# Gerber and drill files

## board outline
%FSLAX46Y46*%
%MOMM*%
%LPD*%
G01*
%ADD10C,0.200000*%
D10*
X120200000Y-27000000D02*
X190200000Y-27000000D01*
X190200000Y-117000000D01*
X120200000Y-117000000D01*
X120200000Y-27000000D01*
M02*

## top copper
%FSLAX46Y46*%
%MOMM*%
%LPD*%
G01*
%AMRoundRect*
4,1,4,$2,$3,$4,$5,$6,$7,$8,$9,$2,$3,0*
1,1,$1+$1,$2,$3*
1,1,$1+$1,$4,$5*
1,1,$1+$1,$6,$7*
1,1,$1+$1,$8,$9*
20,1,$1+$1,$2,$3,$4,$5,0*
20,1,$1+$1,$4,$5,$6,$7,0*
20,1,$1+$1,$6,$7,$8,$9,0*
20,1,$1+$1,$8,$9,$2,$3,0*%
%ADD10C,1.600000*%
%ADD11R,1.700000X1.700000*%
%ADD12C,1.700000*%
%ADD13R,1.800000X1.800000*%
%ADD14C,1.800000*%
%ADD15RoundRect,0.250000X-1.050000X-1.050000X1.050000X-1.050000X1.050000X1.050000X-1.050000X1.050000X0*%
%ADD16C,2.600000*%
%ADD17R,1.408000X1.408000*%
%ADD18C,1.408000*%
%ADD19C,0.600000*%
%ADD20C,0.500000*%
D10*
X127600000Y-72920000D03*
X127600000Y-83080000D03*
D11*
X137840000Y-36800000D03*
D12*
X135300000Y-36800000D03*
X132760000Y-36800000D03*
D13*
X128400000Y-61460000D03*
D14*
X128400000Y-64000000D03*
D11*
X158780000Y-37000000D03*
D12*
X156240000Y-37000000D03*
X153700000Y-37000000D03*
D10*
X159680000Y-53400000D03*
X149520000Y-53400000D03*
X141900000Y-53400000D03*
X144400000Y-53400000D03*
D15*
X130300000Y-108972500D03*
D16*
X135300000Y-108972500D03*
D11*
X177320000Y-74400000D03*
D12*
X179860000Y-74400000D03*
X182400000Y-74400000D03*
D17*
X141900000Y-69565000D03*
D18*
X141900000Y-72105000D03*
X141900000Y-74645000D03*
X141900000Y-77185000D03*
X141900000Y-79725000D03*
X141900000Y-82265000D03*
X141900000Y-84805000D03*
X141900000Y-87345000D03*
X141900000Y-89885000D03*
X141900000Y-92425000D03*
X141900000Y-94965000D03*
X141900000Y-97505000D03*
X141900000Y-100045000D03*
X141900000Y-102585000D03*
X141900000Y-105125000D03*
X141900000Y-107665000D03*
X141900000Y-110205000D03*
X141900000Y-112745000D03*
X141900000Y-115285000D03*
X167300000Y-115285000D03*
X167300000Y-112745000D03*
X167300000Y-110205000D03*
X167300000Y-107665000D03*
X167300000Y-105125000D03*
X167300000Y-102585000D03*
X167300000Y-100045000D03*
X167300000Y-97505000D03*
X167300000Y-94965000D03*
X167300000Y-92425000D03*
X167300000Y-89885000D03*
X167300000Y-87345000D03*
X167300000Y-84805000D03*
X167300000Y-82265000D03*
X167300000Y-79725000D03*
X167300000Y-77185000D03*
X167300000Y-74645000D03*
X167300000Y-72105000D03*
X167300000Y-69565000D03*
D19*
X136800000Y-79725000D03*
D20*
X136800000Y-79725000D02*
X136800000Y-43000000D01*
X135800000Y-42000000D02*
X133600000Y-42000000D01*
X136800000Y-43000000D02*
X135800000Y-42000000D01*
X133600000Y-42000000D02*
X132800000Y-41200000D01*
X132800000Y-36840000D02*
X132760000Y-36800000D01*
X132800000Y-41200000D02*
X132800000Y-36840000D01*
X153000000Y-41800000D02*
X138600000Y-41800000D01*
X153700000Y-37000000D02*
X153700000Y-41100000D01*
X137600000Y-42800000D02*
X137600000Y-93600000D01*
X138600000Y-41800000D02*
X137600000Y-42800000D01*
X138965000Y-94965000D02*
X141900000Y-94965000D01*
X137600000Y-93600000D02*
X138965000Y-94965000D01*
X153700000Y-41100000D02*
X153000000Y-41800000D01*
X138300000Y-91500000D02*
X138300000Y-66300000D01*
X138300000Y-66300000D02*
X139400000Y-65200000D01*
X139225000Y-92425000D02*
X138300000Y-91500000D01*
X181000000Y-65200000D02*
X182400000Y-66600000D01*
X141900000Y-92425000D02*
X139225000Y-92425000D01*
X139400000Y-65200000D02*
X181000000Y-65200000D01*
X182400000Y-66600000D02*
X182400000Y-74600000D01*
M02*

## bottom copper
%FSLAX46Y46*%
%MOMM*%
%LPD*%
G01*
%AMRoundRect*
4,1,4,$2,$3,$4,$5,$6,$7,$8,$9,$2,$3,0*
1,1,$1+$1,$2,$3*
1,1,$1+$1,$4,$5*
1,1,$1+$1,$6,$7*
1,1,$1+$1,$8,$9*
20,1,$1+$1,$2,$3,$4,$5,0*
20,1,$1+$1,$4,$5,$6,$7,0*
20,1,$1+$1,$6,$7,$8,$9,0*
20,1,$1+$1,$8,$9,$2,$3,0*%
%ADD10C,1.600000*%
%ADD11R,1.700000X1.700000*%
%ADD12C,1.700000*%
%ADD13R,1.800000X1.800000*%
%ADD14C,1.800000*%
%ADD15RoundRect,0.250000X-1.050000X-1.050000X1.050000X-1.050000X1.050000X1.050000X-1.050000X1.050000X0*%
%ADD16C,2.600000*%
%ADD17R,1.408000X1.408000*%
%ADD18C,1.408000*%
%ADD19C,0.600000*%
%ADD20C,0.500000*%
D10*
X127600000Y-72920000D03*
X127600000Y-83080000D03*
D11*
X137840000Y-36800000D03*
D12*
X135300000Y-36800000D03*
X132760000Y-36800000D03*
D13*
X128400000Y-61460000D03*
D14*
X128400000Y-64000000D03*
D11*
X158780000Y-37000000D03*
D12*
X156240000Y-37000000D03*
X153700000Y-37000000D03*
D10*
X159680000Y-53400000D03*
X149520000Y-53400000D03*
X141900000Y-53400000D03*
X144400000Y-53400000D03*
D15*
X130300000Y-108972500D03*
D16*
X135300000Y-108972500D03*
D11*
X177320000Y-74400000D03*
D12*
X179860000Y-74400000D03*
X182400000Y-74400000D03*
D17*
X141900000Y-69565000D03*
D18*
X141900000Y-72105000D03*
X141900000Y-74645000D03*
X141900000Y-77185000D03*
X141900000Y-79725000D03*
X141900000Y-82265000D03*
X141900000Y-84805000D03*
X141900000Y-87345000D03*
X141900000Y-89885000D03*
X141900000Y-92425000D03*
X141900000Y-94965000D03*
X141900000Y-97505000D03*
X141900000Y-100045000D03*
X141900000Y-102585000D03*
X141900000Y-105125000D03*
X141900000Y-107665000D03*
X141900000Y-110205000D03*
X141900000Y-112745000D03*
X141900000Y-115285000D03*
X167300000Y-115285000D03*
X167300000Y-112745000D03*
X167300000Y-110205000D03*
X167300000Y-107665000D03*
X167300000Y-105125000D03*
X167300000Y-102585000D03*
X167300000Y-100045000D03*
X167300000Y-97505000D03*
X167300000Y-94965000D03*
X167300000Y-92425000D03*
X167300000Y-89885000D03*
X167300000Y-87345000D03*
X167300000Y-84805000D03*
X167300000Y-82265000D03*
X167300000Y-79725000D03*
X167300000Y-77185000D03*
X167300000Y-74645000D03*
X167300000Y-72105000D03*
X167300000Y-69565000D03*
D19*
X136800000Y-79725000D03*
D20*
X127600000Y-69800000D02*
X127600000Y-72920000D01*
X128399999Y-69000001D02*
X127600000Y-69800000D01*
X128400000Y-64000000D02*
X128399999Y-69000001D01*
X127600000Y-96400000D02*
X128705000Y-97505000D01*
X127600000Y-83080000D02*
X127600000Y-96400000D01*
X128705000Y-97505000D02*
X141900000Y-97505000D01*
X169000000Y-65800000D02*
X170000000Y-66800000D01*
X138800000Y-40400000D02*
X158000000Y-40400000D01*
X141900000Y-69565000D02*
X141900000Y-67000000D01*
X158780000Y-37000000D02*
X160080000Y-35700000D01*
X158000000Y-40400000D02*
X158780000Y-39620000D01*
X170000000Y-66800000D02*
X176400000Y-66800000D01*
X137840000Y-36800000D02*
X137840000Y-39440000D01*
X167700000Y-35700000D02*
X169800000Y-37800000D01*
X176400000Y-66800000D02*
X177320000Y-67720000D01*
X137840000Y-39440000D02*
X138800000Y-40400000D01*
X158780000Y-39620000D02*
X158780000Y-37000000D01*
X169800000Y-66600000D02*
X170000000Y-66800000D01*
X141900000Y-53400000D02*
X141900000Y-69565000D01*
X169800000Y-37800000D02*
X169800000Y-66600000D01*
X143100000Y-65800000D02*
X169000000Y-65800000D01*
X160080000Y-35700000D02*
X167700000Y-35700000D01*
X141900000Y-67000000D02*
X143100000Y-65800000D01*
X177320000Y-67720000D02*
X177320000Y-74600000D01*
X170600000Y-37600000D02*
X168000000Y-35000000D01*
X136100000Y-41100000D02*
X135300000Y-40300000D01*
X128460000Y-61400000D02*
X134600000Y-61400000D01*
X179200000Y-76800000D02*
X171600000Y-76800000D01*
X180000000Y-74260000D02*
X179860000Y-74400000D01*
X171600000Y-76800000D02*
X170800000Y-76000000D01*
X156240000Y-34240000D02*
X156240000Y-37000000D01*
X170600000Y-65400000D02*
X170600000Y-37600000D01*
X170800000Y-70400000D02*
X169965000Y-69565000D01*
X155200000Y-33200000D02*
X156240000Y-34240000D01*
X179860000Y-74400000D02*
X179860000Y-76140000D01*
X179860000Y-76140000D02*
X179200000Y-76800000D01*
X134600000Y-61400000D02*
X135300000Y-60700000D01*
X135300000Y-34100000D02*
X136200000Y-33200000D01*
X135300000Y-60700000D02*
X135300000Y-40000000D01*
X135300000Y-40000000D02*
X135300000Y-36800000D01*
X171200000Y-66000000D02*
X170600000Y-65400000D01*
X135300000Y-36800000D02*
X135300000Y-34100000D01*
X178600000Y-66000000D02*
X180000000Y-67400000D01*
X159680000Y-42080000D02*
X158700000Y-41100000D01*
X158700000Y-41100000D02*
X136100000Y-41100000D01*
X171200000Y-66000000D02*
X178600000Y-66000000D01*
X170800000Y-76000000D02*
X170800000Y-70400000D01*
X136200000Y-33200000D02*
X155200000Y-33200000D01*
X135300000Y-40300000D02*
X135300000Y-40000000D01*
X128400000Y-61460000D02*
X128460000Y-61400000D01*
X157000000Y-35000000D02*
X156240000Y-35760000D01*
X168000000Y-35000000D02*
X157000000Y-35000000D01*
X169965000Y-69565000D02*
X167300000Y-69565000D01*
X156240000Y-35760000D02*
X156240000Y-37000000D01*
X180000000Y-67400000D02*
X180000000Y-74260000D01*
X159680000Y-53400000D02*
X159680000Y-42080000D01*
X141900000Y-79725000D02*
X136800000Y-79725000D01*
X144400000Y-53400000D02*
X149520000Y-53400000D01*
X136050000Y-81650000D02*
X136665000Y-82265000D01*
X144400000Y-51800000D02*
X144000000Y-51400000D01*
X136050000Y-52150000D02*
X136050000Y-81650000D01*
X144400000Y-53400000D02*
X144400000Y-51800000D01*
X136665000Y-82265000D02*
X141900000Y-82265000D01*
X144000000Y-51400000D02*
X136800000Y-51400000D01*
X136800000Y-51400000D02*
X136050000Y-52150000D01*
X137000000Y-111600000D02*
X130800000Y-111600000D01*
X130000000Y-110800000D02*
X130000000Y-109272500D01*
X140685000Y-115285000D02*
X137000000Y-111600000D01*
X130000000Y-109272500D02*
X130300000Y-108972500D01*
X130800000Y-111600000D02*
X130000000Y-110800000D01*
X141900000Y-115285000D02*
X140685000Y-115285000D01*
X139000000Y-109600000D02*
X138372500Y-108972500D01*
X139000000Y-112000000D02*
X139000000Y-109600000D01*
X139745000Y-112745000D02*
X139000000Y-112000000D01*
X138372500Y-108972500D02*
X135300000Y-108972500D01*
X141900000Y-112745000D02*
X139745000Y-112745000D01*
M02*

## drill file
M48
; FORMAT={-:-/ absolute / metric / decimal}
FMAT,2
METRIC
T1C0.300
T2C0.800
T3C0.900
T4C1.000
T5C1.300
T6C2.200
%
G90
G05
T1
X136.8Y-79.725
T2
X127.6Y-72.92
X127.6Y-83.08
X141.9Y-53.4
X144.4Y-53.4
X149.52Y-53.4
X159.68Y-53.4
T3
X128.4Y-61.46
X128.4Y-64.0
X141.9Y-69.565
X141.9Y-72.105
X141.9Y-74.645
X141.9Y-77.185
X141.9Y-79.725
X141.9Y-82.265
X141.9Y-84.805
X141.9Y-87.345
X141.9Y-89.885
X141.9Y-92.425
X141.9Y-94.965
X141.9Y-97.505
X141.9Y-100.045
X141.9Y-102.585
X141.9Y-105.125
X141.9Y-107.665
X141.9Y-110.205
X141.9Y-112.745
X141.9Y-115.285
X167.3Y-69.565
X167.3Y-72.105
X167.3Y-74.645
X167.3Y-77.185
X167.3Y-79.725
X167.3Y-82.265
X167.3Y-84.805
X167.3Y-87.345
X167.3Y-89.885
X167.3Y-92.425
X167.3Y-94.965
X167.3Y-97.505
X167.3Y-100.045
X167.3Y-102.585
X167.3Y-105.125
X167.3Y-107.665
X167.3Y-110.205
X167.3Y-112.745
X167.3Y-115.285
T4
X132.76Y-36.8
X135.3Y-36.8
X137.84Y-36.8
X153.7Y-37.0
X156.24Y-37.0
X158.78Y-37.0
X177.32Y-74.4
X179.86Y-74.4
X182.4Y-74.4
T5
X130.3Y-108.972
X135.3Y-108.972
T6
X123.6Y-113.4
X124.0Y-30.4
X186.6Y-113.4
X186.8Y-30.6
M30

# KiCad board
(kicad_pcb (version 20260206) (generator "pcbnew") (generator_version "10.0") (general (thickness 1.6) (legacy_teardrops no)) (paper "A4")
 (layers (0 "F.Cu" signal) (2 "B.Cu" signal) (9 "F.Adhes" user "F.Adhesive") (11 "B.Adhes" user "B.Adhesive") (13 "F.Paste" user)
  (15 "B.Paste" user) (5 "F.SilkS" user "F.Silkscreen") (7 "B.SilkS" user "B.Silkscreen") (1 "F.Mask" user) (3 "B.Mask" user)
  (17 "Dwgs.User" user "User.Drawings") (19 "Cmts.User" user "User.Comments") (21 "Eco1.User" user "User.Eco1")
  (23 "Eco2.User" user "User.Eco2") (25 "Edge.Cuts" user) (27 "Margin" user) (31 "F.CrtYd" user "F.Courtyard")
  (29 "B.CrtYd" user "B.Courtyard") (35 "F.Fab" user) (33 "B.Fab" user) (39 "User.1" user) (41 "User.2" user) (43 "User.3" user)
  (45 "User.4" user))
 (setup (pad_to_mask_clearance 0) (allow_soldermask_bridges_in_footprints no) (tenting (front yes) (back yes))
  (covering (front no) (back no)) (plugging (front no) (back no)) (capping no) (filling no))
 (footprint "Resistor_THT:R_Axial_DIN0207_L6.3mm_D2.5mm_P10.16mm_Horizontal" (layer "F.Cu") (at 127.6 72.92 -90)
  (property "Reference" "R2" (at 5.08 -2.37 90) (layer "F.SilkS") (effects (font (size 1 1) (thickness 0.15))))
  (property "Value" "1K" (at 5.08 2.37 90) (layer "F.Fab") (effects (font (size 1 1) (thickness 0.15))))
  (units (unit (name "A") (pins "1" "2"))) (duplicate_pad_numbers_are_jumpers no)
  (pad "1" thru_hole circle (at 0 0 270) (size 1.6 1.6) (drill 0.8) (layers "*.Cu" "*.Mask") (remove_unused_layers no) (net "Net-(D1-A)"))
  (pad "2" thru_hole circle (at 10.16 0 270) (size 1.6 1.6) (drill 0.8) (layers "*.Cu" "*.Mask") (remove_unused_layers no)
   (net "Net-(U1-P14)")))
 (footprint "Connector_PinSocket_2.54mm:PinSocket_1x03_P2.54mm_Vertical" (layer "F.Cu") (at 137.84 36.8 -90)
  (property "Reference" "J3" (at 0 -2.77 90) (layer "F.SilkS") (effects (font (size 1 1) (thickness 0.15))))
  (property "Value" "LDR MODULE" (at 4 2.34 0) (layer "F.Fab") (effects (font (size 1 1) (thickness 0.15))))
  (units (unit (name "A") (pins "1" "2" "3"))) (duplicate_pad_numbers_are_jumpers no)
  (pad "1" thru_hole rect (at 0 0 270) (size 1.7 1.7) (drill 1) (layers "*.Cu" "*.Mask") (remove_unused_layers no) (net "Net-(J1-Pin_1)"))
  (pad "2" thru_hole circle (at 0 2.54 270) (size 1.7 1.7) (drill 1) (layers "*.Cu" "*.Mask") (remove_unused_layers no) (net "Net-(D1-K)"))
  (pad "3" thru_hole circle (at 0 5.08 270) (size 1.7 1.7) (drill 1) (layers "*.Cu" "*.Mask") (remove_unused_layers no) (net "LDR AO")))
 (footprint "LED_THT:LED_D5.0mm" (layer "F.Cu") (at 128.4 61.46 -90)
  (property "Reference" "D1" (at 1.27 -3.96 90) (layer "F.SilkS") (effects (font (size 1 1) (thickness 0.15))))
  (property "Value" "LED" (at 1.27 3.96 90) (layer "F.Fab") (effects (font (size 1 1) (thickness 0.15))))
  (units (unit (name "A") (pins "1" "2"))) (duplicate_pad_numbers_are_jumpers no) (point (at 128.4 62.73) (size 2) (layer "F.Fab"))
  (pad "1" thru_hole rect (at 0 0 270) (size 1.8 1.8) (drill 0.9) (layers "*.Cu" "*.Mask") (remove_unused_layers no) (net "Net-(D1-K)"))
  (pad "2" thru_hole circle (at 2.54 0 270) (size 1.8 1.8) (drill 0.9) (layers "*.Cu" "*.Mask") (remove_unused_layers no) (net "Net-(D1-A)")))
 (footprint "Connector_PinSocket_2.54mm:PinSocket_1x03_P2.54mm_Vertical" (layer "F.Cu") (at 158.78 37 -90)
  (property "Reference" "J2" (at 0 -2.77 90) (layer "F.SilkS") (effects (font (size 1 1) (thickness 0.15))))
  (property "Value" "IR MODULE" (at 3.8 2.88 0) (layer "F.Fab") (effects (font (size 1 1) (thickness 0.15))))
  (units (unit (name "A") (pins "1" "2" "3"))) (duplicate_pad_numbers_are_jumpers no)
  (pad "1" thru_hole rect (at 0 0 270) (size 1.7 1.7) (drill 1) (layers "*.Cu" "*.Mask") (remove_unused_layers no) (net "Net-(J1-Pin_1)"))
  (pad "2" thru_hole circle (at 0 2.54 270) (size 1.7 1.7) (drill 1) (layers "*.Cu" "*.Mask") (remove_unused_layers no) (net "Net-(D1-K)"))
  (pad "3" thru_hole circle (at 0 5.08 270) (size 1.7 1.7) (drill 1) (layers "*.Cu" "*.Mask") (remove_unused_layers no) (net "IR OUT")))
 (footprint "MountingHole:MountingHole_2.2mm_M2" (layer "F.Cu") (at 186.6 113.4)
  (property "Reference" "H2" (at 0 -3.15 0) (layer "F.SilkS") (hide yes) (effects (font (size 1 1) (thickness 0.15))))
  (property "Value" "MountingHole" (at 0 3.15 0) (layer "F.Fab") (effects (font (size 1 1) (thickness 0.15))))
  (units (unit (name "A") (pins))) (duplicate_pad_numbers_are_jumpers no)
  (pad "" np_thru_hole circle (at 0 0) (size 2.2 2.2) (drill 2.2) (layers "*.Cu" "*.Mask")))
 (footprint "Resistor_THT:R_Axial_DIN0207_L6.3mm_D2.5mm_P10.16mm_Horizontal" (layer "F.Cu") (at 159.68 53.4 180)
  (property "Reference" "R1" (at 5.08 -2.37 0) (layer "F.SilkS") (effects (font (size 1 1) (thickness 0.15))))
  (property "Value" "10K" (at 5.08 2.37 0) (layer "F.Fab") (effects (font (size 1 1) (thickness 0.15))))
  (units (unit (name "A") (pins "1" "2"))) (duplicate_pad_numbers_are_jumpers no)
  (pad "1" thru_hole circle (at 0 0 180) (size 1.6 1.6) (drill 0.8) (layers "*.Cu" "*.Mask") (remove_unused_layers no) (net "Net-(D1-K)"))
  (pad "2" thru_hole circle (at 10.16 0 180) (size 1.6 1.6) (drill 0.8) (layers "*.Cu" "*.Mask") (remove_unused_layers no) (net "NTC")))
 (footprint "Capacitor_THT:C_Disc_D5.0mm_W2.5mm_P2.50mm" (layer "F.Cu") (at 141.9 53.4)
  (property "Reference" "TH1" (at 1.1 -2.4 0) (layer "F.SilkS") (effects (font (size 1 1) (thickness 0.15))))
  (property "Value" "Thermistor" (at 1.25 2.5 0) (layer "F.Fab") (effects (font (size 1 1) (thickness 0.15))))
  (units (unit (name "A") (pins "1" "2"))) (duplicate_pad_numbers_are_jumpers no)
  (pad "1" thru_hole circle (at 0 0) (size 1.6 1.6) (drill 0.8) (layers "*.Cu" "*.Mask") (remove_unused_layers no) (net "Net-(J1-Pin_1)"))
  (pad "2" thru_hole circle (at 2.5 0) (size 1.6 1.6) (drill 0.8) (layers "*.Cu" "*.Mask") (remove_unused_layers no) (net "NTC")))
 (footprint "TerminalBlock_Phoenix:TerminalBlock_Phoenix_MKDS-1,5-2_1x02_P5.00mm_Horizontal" (layer "F.Cu") (at 130.3 108.9725)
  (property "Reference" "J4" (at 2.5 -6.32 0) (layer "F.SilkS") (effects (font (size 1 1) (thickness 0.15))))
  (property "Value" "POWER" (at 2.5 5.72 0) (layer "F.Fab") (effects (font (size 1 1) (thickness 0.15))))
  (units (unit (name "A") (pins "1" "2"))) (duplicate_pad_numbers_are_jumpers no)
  (pad "1" thru_hole roundrect (at 0 0) (size 2.6 2.6) (drill 1.3) (layers "*.Cu" "*.Mask") (remove_unused_layers no)
   (roundrect_rratio 0.096154) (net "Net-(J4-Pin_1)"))
  (pad "2" thru_hole circle (at 5 0) (size 2.6 2.6) (drill 1.3) (layers "*.Cu" "*.Mask") (remove_unused_layers no) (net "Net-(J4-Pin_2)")))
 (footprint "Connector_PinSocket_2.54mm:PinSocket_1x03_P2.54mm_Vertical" (layer "F.Cu") (at 177.32 74.4 90)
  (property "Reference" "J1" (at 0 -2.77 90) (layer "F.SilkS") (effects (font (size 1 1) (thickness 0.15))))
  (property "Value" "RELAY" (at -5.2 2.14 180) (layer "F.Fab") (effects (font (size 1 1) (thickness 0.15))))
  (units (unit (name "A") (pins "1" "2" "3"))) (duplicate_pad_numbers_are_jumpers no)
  (pad "1" thru_hole rect (at 0 0 90) (size 1.7 1.7) (drill 1) (layers "*.Cu" "*.Mask") (remove_unused_layers no) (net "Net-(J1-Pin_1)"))
  (pad "2" thru_hole circle (at 0 2.54 90) (size 1.7 1.7) (drill 1) (layers "*.Cu" "*.Mask") (remove_unused_layers no) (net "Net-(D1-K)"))
  (pad "3" thru_hole circle (at 0 5.08 90) (size 1.7 1.7) (drill 1) (layers "*.Cu" "*.Mask") (remove_unused_layers no) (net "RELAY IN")))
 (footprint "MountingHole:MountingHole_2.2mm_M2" (layer "F.Cu") (at 186.8 30.6)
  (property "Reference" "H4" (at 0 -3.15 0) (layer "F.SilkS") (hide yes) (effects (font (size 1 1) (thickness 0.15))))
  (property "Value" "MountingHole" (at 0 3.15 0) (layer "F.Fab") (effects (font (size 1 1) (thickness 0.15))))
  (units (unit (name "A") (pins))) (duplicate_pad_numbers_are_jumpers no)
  (pad "" np_thru_hole circle (at 0 0) (size 2.2 2.2) (drill 2.2) (layers "*.Cu" "*.Mask")))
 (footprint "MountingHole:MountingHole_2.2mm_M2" (layer "F.Cu") (at 124 30.4)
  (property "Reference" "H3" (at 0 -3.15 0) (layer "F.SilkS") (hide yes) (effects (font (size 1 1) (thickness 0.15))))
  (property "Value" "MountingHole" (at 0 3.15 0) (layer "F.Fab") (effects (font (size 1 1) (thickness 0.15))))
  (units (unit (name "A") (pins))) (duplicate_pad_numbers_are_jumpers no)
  (pad "" np_thru_hole circle (at 0 0) (size 2.2 2.2) (drill 2.2) (layers "*.Cu" "*.Mask")))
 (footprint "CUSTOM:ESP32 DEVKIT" (layer "F.Cu") (at 154.57 93.21)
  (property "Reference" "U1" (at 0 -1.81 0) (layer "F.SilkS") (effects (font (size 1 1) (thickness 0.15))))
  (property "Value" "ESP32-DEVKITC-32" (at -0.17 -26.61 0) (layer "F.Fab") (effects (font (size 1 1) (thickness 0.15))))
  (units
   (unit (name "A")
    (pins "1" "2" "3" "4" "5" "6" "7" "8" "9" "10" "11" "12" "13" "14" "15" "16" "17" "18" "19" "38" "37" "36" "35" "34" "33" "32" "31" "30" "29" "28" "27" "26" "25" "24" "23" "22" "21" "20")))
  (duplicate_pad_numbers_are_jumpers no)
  (pad "1" thru_hole rect (at -12.67 -23.645) (size 1.408 1.408) (drill 0.9) (layers "*.Cu" "*.Mask") (remove_unused_layers no)
   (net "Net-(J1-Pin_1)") (solder_mask_margin 0.102))
  (pad "2" thru_hole circle (at -12.67 -21.105) (size 1.408 1.408) (drill 0.9) (layers "*.Cu" "*.Mask") (remove_unused_layers no)
   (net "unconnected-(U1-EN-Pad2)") (solder_mask_margin 0.102))
  (pad "3" thru_hole circle (at -12.67 -18.565) (size 1.408 1.408) (drill 0.9) (layers "*.Cu" "*.Mask") (remove_unused_layers no)
   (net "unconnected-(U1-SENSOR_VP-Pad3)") (solder_mask_margin 0.102))
  (pad "4" thru_hole circle (at -12.67 -16.025) (size 1.408 1.408) (drill 0.9) (layers "*.Cu" "*.Mask") (remove_unused_layers no)
   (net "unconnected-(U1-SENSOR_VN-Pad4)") (solder_mask_margin 0.102))
  (pad "5" thru_hole circle (at -12.67 -13.485) (size 1.408 1.408) (drill 0.9) (layers "*.Cu" "*.Mask") (remove_unused_layers no)
   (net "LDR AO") (solder_mask_margin 0.102))
  (pad "6" thru_hole circle (at -12.67 -10.945) (size 1.408 1.408) (drill 0.9) (layers "*.Cu" "*.Mask") (remove_unused_layers no)
   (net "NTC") (solder_mask_margin 0.102))
  (pad "7" thru_hole circle (at -12.67 -8.405) (size 1.408 1.408) (drill 0.9) (layers "*.Cu" "*.Mask") (remove_unused_layers no)
   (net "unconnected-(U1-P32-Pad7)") (solder_mask_margin 0.102))
  (pad "8" thru_hole circle (at -12.67 -5.865) (size 1.408 1.408) (drill 0.9) (layers "*.Cu" "*.Mask") (remove_unused_layers no)
   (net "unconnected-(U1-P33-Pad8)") (solder_mask_margin 0.102))
  (pad "9" thru_hole circle (at -12.67 -3.325) (size 1.408 1.408) (drill 0.9) (layers "*.Cu" "*.Mask") (remove_unused_layers no)
   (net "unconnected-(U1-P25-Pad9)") (solder_mask_margin 0.102))
  (pad "10" thru_hole circle (at -12.67 -0.785) (size 1.408 1.408) (drill 0.9) (layers "*.Cu" "*.Mask") (remove_unused_layers no)
   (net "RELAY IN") (solder_mask_margin 0.102))
  (pad "11" thru_hole circle (at -12.67 1.755) (size 1.408 1.408) (drill 0.9) (layers "*.Cu" "*.Mask") (remove_unused_layers no)
   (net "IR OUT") (solder_mask_margin 0.102))
  (pad "12" thru_hole circle (at -12.67 4.295) (size 1.408 1.408) (drill 0.9) (layers "*.Cu" "*.Mask") (remove_unused_layers no)
   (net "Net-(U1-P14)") (solder_mask_margin 0.102))
  (pad "13" thru_hole circle (at -12.67 6.835) (size 1.408 1.408) (drill 0.9) (layers "*.Cu" "*.Mask") (remove_unused_layers no)
   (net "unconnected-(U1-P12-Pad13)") (solder_mask_margin 0.102))
  (pad "14" thru_hole circle (at -12.67 9.375) (size 1.408 1.408) (drill 0.9) (layers "*.Cu" "*.Mask") (remove_unused_layers no)
   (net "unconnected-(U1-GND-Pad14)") (solder_mask_margin 0.102))
  (pad "15" thru_hole circle (at -12.67 11.915) (size 1.408 1.408) (drill 0.9) (layers "*.Cu" "*.Mask") (remove_unused_layers no)
   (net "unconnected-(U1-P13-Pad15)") (solder_mask_margin 0.102))
  (pad "16" thru_hole circle (at -12.67 14.455) (size 1.408 1.408) (drill 0.9) (layers "*.Cu" "*.Mask") (remove_unused_layers no)
   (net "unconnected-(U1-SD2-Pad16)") (solder_mask_margin 0.102))
  (pad "17" thru_hole circle (at -12.67 16.995) (size 1.408 1.408) (drill 0.9) (layers "*.Cu" "*.Mask") (remove_unused_layers no)
   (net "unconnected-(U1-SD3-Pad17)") (solder_mask_margin 0.102))
  (pad "18" thru_hole circle (at -12.67 19.535) (size 1.408 1.408) (drill 0.9) (layers "*.Cu" "*.Mask") (remove_unused_layers no)
   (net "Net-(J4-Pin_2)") (solder_mask_margin 0.102))
  (pad "19" thru_hole circle (at -12.67 22.075) (size 1.408 1.408) (drill 0.9) (layers "*.Cu" "*.Mask") (remove_unused_layers no)
   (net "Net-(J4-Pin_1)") (solder_mask_margin 0.102))
  (pad "20" thru_hole circle (at 12.73 22.075) (size 1.408 1.408) (drill 0.9) (layers "*.Cu" "*.Mask") (remove_unused_layers no)
   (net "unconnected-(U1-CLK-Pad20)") (solder_mask_margin 0.102))
  (pad "21" thru_hole circle (at 12.73 19.535) (size 1.408 1.408) (drill 0.9) (layers "*.Cu" "*.Mask") (remove_unused_layers no)
   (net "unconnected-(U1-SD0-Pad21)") (solder_mask_margin 0.102))
  (pad "22" thru_hole circle (at 12.73 16.995) (size 1.408 1.408) (drill 0.9) (layers "*.Cu" "*.Mask") (remove_unused_layers no)
   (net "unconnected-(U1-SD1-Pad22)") (solder_mask_margin 0.102))
  (pad "23" thru_hole circle (at 12.73 14.455) (size 1.408 1.408) (drill 0.9) (layers "*.Cu" "*.Mask") (remove_unused_layers no)
   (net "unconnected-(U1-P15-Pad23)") (solder_mask_margin 0.102))
  (pad "24" thru_hole circle (at 12.73 11.915) (size 1.408 1.408) (drill 0.9) (layers "*.Cu" "*.Mask") (remove_unused_layers no)
   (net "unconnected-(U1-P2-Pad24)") (solder_mask_margin 0.102))
  (pad "25" thru_hole circle (at 12.73 9.375) (size 1.408 1.408) (drill 0.9) (layers "*.Cu" "*.Mask") (remove_unused_layers no)
   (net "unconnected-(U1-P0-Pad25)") (solder_mask_margin 0.102))
  (pad "26" thru_hole circle (at 12.73 6.835) (size 1.408 1.408) (drill 0.9) (layers "*.Cu" "*.Mask") (remove_unused_layers no)
   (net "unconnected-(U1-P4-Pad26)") (solder_mask_margin 0.102))
  (pad "27" thru_hole circle (at 12.73 4.295) (size 1.408 1.408) (drill 0.9) (layers "*.Cu" "*.Mask") (remove_unused_layers no)
   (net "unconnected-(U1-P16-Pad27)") (solder_mask_margin 0.102))
  (pad "28" thru_hole circle (at 12.73 1.755) (size 1.408 1.408) (drill 0.9) (layers "*.Cu" "*.Mask") (remove_unused_layers no)
   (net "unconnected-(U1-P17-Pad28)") (solder_mask_margin 0.102))
  (pad "29" thru_hole circle (at 12.73 -0.785) (size 1.408 1.408) (drill 0.9) (layers "*.Cu" "*.Mask") (remove_unused_layers no)
   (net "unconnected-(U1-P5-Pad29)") (solder_mask_margin 0.102))
  (pad "30" thru_hole circle (at 12.73 -3.325) (size 1.408 1.408) (drill 0.9) (layers "*.Cu" "*.Mask") (remove_unused_layers no)
   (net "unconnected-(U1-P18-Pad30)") (solder_mask_margin 0.102))
  (pad "31" thru_hole circle (at 12.73 -5.865) (size 1.408 1.408) (drill 0.9) (layers "*.Cu" "*.Mask") (remove_unused_layers no)
   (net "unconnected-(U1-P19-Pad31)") (solder_mask_margin 0.102))
  (pad "32" thru_hole circle (at 12.73 -8.405) (size 1.408 1.408) (drill 0.9) (layers "*.Cu" "*.Mask") (remove_unused_layers no)
   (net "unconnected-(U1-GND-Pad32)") (solder_mask_margin 0.102))
  (pad "33" thru_hole circle (at 12.73 -10.945) (size 1.408 1.408) (drill 0.9) (layers "*.Cu" "*.Mask") (remove_unused_layers no)
   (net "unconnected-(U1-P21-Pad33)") (solder_mask_margin 0.102))
  (pad "34" thru_hole circle (at 12.73 -13.485) (size 1.408 1.408) (drill 0.9) (layers "*.Cu" "*.Mask") (remove_unused_layers no)
   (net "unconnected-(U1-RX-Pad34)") (solder_mask_margin 0.102))
  (pad "35" thru_hole circle (at 12.73 -16.025) (size 1.408 1.408) (drill 0.9) (layers "*.Cu" "*.Mask") (remove_unused_layers no)
   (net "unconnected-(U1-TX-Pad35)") (solder_mask_margin 0.102))
  (pad "36" thru_hole circle (at 12.73 -18.565) (size 1.408 1.408) (drill 0.9) (layers "*.Cu" "*.Mask") (remove_unused_layers no)
   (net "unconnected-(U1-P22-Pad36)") (solder_mask_margin 0.102))
  (pad "37" thru_hole circle (at 12.73 -21.105) (size 1.408 1.408) (drill 0.9) (layers "*.Cu" "*.Mask") (remove_unused_layers no)
   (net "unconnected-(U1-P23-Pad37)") (solder_mask_margin 0.102))
  (pad "38" thru_hole circle (at 12.73 -23.645) (size 1.408 1.408) (drill 0.9) (layers "*.Cu" "*.Mask") (remove_unused_layers no)
   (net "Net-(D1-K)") (solder_mask_margin 0.102)))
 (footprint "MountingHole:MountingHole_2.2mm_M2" (layer "F.Cu") (at 123.6 113.4)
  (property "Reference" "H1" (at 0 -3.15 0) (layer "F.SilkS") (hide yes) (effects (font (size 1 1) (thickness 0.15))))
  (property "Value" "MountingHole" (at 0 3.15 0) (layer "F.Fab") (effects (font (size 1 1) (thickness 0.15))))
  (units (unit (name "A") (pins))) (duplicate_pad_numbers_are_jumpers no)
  (pad "" np_thru_hole circle (at 0 0) (size 2.2 2.2) (drill 2.2) (layers "*.Cu" "*.Mask")))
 (gr_rect (start 120.2 27) (end 190.2 117) (stroke (width 0.2) (type solid)) (fill no) (layer "Edge.Cuts"))
 (segment (start 127.6 69.8) (end 127.6 72.92) (width 0.5) (layer "B.Cu") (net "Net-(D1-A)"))
 (segment (start 128.399999 69.000001) (end 127.6 69.8) (width 0.5) (layer "B.Cu") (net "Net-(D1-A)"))
 (segment (start 128.4 64) (end 128.399999 69.000001) (width 0.5) (layer "B.Cu") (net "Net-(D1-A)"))
 (segment (start 127.6 96.4) (end 128.705 97.505) (width 0.5) (layer "B.Cu") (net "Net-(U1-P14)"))
 (segment (start 127.6 83.08) (end 127.6 96.4) (width 0.5) (layer "B.Cu") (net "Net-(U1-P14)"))
 (segment (start 128.705 97.505) (end 141.9 97.505) (width 0.5) (layer "B.Cu") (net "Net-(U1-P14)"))
 (segment (start 169 65.8) (end 170 66.8) (width 0.5) (layer "B.Cu") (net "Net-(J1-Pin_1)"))
 (segment (start 138.8 40.4) (end 158 40.4) (width 0.5) (layer "B.Cu") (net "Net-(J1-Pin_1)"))
 (segment (start 141.9 69.565) (end 141.9 67) (width 0.5) (layer "B.Cu") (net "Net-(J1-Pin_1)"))
 (segment (start 158.78 37) (end 160.08 35.7) (width 0.5) (layer "B.Cu") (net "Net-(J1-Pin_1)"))
 (segment (start 158 40.4) (end 158.78 39.62) (width 0.5) (layer "B.Cu") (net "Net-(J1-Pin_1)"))
 (segment (start 170 66.8) (end 176.4 66.8) (width 0.5) (layer "B.Cu") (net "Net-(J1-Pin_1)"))
 (segment (start 137.84 36.8) (end 137.84 39.44) (width 0.5) (layer "B.Cu") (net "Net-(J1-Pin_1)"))
 (segment (start 167.7 35.7) (end 169.8 37.8) (width 0.5) (layer "B.Cu") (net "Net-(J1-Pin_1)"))
 (segment (start 176.4 66.8) (end 177.32 67.72) (width 0.5) (layer "B.Cu") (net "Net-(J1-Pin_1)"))
 (segment (start 137.84 39.44) (end 138.8 40.4) (width 0.5) (layer "B.Cu") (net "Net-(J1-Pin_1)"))
 (segment (start 158.78 39.62) (end 158.78 37) (width 0.5) (layer "B.Cu") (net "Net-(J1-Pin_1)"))
 (segment (start 169.8 66.6) (end 170 66.8) (width 0.5) (layer "B.Cu") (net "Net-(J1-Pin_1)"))
 (segment (start 141.9 53.4) (end 141.9 69.565) (width 0.5) (layer "B.Cu") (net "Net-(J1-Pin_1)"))
 (segment (start 169.8 37.8) (end 169.8 66.6) (width 0.5) (layer "B.Cu") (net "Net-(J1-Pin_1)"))
 (segment (start 143.1 65.8) (end 169 65.8) (width 0.5) (layer "B.Cu") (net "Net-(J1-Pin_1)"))
 (segment (start 160.08 35.7) (end 167.7 35.7) (width 0.5) (layer "B.Cu") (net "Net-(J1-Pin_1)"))
 (segment (start 141.9 67) (end 143.1 65.8) (width 0.5) (layer "B.Cu") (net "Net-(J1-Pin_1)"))
 (segment (start 177.32 67.72) (end 177.32 74.6) (width 0.5) (layer "B.Cu") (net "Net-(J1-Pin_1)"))
 (segment (start 170.6 37.6) (end 168 35) (width 0.5) (layer "B.Cu") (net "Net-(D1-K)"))
 (segment (start 136.1 41.1) (end 135.3 40.3) (width 0.5) (layer "B.Cu") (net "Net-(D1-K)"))
 (segment (start 128.46 61.4) (end 134.6 61.4) (width 0.5) (layer "B.Cu") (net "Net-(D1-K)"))
 (segment (start 179.2 76.8) (end 171.6 76.8) (width 0.5) (layer "B.Cu") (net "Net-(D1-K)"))
 (segment (start 180 74.26) (end 179.86 74.4) (width 0.5) (layer "B.Cu") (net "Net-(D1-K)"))
 (segment (start 171.6 76.8) (end 170.8 76) (width 0.5) (layer "B.Cu") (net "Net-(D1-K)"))
 (segment (start 156.24 34.24) (end 156.24 37) (width 0.5) (layer "B.Cu") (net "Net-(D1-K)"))
 (segment (start 170.6 65.4) (end 170.6 37.6) (width 0.5) (layer "B.Cu") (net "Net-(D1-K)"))
 (segment (start 170.8 70.4) (end 169.965 69.565) (width 0.5) (layer "B.Cu") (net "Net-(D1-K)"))
 (segment (start 155.2 33.2) (end 156.24 34.24) (width 0.5) (layer "B.Cu") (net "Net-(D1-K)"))
 (segment (start 179.86 74.4) (end 179.86 76.14) (width 0.5) (layer "B.Cu") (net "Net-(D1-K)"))
 (segment (start 179.86 76.14) (end 179.2 76.8) (width 0.5) (layer "B.Cu") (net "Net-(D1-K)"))
 (segment (start 134.6 61.4) (end 135.3 60.7) (width 0.5) (layer "B.Cu") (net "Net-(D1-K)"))
 (segment (start 135.3 34.1) (end 136.2 33.2) (width 0.5) (layer "B.Cu") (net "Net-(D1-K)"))
 (segment (start 135.3 60.7) (end 135.3 40) (width 0.5) (layer "B.Cu") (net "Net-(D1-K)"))
 (segment (start 135.3 40) (end 135.3 36.8) (width 0.5) (layer "B.Cu") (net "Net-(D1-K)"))
 (segment (start 171.2 66) (end 170.6 65.4) (width 0.5) (layer "B.Cu") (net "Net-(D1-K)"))
 (segment (start 135.3 36.8) (end 135.3 34.1) (width 0.5) (layer "B.Cu") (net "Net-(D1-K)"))
 (segment (start 178.6 66) (end 180 67.4) (width 0.5) (layer "B.Cu") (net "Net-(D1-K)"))
 (segment (start 159.68 42.08) (end 158.7 41.1) (width 0.5) (layer "B.Cu") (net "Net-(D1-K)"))
 (segment (start 158.7 41.1) (end 136.1 41.1) (width 0.5) (layer "B.Cu") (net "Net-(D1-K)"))
 (segment (start 171.2 66) (end 178.6 66) (width 0.5) (layer "B.Cu") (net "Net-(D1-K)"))
 (segment (start 170.8 76) (end 170.8 70.4) (width 0.5) (layer "B.Cu") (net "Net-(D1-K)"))
 (segment (start 136.2 33.2) (end 155.2 33.2) (width 0.5) (layer "B.Cu") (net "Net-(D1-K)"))
 (segment (start 135.3 40.3) (end 135.3 40) (width 0.5) (layer "B.Cu") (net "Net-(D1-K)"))
 (segment (start 128.4 61.46) (end 128.46 61.4) (width 0.5) (layer "B.Cu") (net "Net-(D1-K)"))
 (segment (start 157 35) (end 156.24 35.76) (width 0.5) (layer "B.Cu") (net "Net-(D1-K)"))
 (segment (start 168 35) (end 157 35) (width 0.5) (layer "B.Cu") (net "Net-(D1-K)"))
 (segment (start 169.965 69.565) (end 167.3 69.565) (width 0.5) (layer "B.Cu") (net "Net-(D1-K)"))
 (segment (start 156.24 35.76) (end 156.24 37) (width 0.5) (layer "B.Cu") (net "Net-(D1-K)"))
 (segment (start 180 67.4) (end 180 74.26) (width 0.5) (layer "B.Cu") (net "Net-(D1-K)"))
 (segment (start 159.68 53.4) (end 159.68 42.08) (width 0.5) (layer "B.Cu") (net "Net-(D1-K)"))
 (segment (start 136.8 79.725) (end 136.8 43) (width 0.5) (layer "F.Cu") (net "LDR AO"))
 (segment (start 135.8 42) (end 133.6 42) (width 0.5) (layer "F.Cu") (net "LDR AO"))
 (segment (start 136.8 43) (end 135.8 42) (width 0.5) (layer "F.Cu") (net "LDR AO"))
 (segment (start 133.6 42) (end 132.8 41.2) (width 0.5) (layer "F.Cu") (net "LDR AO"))
 (segment (start 132.8 36.84) (end 132.76 36.8) (width 0.5) (layer "F.Cu") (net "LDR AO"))
 (segment (start 132.8 41.2) (end 132.8 36.84) (width 0.5) (layer "F.Cu") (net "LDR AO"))
 (via (at 136.8 79.725) (size 0.6) (drill 0.3) (layers "F.Cu" "B.Cu") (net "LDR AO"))
 (segment (start 141.9 79.725) (end 136.8 79.725) (width 0.5) (layer "B.Cu") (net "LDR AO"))
 (segment (start 153 41.8) (end 138.6 41.8) (width 0.5) (layer "F.Cu") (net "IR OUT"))
 (segment (start 153.7 37) (end 153.7 41.1) (width 0.5) (layer "F.Cu") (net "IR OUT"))
 (segment (start 137.6 42.8) (end 137.6 93.6) (width 0.5) (layer "F.Cu") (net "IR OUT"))
 (segment (start 138.6 41.8) (end 137.6 42.8) (width 0.5) (layer "F.Cu") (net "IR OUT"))
 (segment (start 138.965 94.965) (end 141.9 94.965) (width 0.5) (layer "F.Cu") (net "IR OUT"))
 (segment (start 137.6 93.6) (end 138.965 94.965) (width 0.5) (layer "F.Cu") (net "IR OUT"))
 (segment (start 153.7 41.1) (end 153 41.8) (width 0.5) (layer "F.Cu") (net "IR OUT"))
 (segment (start 144.4 53.4) (end 149.52 53.4) (width 0.5) (layer "B.Cu") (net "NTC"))
 (segment (start 136.05 81.65) (end 136.665 82.265) (width 0.5) (layer "B.Cu") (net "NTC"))
 (segment (start 144.4 51.8) (end 144 51.4) (width 0.5) (layer "B.Cu") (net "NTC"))
 (segment (start 136.05 52.15) (end 136.05 81.65) (width 0.5) (layer "B.Cu") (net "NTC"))
 (segment (start 144.4 53.4) (end 144.4 51.8) (width 0.5) (layer "B.Cu") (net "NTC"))
 (segment (start 136.665 82.265) (end 141.9 82.265) (width 0.5) (layer "B.Cu") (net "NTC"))
 (segment (start 144 51.4) (end 136.8 51.4) (width 0.5) (layer "B.Cu") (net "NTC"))
 (segment (start 136.8 51.4) (end 136.05 52.15) (width 0.5) (layer "B.Cu") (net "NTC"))
 (segment (start 137 111.6) (end 130.8 111.6) (width 0.5) (layer "B.Cu") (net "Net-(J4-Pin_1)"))
 (segment (start 130 110.8) (end 130 109.2725) (width 0.5) (layer "B.Cu") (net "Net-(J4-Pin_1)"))
 (segment (start 140.685 115.285) (end 137 111.6) (width 0.5) (layer "B.Cu") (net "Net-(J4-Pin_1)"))
 (segment (start 130 109.2725) (end 130.3 108.9725) (width 0.5) (layer "B.Cu") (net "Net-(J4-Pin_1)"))
 (segment (start 130.8 111.6) (end 130 110.8) (width 0.5) (layer "B.Cu") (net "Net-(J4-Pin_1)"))
 (segment (start 141.9 115.285) (end 140.685 115.285) (width 0.5) (layer "B.Cu") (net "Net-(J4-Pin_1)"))
 (segment (start 139 109.6) (end 138.3725 108.9725) (width 0.5) (layer "B.Cu") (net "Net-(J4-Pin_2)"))
 (segment (start 139 112) (end 139 109.6) (width 0.5) (layer "B.Cu") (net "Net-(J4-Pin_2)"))
 (segment (start 139.745 112.745) (end 139 112) (width 0.5) (layer "B.Cu") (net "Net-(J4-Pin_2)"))
 (segment (start 138.3725 108.9725) (end 135.3 108.9725) (width 0.5) (layer "B.Cu") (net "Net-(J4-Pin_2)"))
 (segment (start 141.9 112.745) (end 139.745 112.745) (width 0.5) (layer "B.Cu") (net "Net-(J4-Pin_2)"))
 (segment (start 138.3 91.5) (end 138.3 66.3) (width 0.5) (layer "F.Cu") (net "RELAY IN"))
 (segment (start 138.3 66.3) (end 139.4 65.2) (width 0.5) (layer "F.Cu") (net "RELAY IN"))
 (segment (start 139.225 92.425) (end 138.3 91.5) (width 0.5) (layer "F.Cu") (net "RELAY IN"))
 (segment (start 181 65.2) (end 182.4 66.6) (width 0.5) (layer "F.Cu") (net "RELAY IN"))
 (segment (start 141.9 92.425) (end 139.225 92.425) (width 0.5) (layer "F.Cu") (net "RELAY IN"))
 (segment (start 139.4 65.2) (end 181 65.2) (width 0.5) (layer "F.Cu") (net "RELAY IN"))
 (segment (start 182.4 66.6) (end 182.4 74.6) (width 0.5) (layer "F.Cu") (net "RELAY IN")))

